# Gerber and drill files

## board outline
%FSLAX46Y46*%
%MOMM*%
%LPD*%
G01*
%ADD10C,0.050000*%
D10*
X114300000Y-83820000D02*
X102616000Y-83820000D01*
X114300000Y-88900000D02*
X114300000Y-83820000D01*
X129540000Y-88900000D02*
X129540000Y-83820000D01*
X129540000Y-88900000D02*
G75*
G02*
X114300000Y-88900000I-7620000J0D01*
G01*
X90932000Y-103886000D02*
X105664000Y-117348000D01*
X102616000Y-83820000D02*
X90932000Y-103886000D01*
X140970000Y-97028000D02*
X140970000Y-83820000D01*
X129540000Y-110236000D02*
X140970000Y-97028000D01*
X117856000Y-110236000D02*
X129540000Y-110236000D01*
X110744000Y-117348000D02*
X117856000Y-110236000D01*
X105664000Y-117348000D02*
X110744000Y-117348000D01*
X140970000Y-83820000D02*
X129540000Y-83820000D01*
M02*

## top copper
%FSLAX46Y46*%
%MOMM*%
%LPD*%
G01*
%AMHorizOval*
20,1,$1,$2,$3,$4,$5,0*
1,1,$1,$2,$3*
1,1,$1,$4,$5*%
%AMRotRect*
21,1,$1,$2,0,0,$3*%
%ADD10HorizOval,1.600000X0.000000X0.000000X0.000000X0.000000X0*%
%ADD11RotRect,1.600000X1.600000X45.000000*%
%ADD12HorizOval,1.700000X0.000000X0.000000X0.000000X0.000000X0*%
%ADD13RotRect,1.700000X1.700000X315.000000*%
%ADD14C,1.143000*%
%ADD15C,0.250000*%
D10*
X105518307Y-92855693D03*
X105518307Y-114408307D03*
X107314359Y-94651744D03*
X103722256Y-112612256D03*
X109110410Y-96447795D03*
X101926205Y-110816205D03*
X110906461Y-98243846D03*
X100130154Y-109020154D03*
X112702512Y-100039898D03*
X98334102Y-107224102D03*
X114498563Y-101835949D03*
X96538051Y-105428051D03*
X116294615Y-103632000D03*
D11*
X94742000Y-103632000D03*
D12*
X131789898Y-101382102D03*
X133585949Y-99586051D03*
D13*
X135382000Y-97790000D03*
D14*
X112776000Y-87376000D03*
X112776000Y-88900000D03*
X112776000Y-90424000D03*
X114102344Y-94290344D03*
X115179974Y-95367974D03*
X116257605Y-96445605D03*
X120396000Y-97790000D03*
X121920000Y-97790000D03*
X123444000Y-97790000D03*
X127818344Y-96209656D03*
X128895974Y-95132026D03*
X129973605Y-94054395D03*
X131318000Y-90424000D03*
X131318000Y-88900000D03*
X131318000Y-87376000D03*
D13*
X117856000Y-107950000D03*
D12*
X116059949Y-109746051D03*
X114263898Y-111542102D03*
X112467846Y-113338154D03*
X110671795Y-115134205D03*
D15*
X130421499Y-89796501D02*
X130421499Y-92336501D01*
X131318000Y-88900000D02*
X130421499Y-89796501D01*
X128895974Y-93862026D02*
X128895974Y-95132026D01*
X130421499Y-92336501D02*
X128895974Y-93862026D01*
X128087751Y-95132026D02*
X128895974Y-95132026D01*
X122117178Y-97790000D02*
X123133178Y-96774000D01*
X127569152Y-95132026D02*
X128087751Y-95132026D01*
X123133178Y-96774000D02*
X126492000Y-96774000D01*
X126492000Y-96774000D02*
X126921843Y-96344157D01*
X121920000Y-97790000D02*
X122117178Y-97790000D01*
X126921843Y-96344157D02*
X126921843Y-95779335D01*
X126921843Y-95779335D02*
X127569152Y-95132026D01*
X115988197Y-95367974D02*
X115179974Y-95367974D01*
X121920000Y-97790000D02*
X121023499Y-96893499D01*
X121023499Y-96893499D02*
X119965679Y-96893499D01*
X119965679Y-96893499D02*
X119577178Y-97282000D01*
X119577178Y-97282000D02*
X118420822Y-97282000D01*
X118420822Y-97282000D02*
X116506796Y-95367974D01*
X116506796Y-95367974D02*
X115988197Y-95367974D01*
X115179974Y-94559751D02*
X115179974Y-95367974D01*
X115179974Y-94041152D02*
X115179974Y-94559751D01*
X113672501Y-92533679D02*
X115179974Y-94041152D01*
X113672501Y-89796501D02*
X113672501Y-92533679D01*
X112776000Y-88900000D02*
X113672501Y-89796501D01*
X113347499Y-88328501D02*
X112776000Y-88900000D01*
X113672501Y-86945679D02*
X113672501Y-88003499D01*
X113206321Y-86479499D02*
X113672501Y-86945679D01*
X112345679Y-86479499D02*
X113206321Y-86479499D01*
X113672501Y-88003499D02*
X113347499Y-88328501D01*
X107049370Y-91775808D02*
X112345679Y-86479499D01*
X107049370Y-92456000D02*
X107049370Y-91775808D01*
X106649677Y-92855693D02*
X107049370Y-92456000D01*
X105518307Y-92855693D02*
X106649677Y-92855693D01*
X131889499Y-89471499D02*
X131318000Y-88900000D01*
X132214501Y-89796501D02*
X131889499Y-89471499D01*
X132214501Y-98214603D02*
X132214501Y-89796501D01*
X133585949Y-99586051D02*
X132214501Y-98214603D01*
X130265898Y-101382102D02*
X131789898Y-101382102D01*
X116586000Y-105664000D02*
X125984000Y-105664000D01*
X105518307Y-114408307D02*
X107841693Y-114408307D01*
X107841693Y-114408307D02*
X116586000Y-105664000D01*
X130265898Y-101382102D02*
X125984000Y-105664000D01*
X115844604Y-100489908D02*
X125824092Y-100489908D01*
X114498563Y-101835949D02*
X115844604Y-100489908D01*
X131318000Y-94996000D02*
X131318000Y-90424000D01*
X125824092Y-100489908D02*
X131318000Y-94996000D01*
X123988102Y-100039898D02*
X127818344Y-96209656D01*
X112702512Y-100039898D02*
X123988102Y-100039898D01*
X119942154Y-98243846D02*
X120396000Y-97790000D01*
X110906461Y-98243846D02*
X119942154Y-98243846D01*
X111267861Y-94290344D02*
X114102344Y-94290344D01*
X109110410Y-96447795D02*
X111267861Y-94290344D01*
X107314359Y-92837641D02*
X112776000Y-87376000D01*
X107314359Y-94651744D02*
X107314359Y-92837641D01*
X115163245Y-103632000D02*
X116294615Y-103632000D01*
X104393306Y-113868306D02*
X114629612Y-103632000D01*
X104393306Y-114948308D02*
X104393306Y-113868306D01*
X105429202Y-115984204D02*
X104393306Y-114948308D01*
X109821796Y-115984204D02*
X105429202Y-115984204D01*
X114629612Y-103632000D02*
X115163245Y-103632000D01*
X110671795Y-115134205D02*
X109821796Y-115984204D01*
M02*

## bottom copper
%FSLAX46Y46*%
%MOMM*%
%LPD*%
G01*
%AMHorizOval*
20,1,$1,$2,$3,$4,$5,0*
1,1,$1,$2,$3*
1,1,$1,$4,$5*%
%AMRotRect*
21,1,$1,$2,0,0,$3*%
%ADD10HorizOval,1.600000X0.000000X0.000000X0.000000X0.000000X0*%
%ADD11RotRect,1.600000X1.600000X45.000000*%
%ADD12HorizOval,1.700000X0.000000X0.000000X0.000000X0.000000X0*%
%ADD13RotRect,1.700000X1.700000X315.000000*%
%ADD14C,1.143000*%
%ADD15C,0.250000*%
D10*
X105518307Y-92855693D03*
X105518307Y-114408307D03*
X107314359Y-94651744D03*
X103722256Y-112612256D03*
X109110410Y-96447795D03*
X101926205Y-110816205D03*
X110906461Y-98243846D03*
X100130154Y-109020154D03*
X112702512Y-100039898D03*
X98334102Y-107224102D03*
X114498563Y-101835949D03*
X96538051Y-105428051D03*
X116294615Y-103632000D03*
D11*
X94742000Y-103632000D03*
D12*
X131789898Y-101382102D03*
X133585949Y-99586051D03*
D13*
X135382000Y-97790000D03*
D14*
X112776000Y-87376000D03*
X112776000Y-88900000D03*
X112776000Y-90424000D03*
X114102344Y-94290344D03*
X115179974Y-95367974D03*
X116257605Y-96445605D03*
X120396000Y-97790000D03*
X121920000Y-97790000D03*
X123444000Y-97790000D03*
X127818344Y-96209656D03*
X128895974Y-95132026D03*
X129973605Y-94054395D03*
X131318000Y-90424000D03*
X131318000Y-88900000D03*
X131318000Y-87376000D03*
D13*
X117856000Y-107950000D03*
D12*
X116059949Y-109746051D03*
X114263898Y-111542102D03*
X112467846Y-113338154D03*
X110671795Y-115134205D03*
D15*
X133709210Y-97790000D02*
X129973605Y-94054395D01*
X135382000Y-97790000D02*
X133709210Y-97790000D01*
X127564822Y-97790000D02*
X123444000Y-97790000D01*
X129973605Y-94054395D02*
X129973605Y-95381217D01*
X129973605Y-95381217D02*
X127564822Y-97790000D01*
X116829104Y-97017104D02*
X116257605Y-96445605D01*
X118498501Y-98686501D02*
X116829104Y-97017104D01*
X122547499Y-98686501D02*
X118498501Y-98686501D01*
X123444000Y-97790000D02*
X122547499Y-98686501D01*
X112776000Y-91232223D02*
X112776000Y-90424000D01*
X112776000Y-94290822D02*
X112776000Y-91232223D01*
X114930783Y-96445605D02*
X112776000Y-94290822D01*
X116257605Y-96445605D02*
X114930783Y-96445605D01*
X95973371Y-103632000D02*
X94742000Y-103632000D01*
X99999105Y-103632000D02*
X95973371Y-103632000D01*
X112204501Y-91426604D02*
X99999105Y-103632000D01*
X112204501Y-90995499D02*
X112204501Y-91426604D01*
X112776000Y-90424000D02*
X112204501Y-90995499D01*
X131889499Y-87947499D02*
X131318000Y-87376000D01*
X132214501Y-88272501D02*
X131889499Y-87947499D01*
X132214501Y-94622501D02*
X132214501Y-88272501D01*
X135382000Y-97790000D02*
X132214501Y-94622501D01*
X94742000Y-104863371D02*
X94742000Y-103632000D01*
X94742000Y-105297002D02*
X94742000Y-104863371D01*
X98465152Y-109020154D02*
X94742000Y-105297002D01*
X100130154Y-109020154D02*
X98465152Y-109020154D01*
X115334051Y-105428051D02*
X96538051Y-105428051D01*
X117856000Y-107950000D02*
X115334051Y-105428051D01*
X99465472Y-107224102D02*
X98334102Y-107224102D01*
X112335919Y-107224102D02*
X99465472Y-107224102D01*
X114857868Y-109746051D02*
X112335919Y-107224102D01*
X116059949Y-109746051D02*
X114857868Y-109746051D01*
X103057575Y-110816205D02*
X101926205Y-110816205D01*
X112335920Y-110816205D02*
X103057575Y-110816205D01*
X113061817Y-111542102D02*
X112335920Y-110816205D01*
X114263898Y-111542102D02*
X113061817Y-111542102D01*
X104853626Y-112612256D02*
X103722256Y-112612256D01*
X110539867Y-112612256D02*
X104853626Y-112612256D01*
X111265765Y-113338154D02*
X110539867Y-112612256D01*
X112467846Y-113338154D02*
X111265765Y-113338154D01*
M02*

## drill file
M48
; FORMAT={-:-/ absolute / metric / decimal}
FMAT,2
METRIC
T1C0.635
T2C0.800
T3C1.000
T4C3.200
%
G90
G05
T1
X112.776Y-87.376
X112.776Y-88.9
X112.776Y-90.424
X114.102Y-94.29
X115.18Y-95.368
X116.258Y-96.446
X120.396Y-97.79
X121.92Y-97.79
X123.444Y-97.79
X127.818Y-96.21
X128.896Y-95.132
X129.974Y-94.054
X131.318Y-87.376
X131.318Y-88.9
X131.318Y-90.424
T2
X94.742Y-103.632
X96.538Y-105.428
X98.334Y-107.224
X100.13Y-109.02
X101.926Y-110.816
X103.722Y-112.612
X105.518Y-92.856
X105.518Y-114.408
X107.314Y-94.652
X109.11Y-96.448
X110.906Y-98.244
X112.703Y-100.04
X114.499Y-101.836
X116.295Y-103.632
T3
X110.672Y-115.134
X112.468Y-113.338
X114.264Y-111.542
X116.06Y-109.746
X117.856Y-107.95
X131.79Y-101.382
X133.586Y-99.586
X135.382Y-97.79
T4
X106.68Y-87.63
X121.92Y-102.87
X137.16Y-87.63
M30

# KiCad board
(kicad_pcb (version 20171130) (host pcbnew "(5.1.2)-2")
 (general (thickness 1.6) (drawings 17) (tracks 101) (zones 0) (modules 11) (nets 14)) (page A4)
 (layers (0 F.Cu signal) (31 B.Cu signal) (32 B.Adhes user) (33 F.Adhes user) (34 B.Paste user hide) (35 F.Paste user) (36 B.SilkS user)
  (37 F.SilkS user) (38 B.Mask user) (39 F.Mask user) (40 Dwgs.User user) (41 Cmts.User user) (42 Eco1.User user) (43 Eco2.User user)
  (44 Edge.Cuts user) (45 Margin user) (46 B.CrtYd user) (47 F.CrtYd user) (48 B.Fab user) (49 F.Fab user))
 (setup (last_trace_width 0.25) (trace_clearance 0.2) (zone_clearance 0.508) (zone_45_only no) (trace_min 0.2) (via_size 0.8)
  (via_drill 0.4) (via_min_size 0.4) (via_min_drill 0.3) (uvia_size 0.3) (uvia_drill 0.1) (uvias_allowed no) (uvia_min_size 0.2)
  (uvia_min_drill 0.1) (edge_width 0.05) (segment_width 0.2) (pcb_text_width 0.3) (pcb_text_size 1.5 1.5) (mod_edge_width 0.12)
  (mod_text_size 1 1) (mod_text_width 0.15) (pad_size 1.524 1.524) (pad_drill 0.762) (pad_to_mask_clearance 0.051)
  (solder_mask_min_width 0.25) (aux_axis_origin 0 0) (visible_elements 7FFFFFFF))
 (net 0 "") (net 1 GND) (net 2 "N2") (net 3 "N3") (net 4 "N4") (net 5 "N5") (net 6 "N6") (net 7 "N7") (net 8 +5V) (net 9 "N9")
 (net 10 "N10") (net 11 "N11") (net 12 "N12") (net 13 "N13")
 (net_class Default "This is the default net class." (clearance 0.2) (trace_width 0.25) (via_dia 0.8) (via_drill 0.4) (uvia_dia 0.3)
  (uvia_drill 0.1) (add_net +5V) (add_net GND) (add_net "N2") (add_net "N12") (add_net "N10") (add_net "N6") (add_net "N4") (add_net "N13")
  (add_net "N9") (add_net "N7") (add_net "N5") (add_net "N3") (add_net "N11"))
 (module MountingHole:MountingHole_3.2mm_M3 (layer F.Cu) (at 121.92 102.87)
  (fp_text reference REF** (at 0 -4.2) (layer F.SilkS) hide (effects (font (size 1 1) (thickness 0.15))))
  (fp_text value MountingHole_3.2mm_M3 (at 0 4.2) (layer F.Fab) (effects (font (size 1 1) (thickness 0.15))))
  (pad 1 np_thru_hole circle (at 0 0) (size 3.2 3.2) (drill 3.2) (layers *.Cu *.Mask)))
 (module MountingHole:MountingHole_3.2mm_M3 (layer F.Cu) (at 137.16 87.63)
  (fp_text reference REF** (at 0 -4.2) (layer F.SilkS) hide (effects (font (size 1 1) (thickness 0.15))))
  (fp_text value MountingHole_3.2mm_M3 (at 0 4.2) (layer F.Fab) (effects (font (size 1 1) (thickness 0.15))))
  (pad 1 np_thru_hole circle (at 0 0) (size 3.2 3.2) (drill 3.2) (layers *.Cu *.Mask)))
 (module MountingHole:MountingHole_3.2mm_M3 (layer F.Cu) (at 106.68 87.63)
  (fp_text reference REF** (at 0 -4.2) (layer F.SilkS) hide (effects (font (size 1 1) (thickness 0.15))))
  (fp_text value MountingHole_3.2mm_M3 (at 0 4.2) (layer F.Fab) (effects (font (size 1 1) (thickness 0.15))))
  (pad 1 np_thru_hole circle (at 0 0) (size 3.2 3.2) (drill 3.2) (layers *.Cu *.Mask)))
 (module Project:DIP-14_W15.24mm (layer F.Cu) (at 94.742 103.632 45)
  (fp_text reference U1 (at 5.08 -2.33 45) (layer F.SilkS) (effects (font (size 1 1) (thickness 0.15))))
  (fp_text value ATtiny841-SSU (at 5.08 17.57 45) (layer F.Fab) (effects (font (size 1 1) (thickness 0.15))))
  (pad 14 thru_hole oval (at 15.24 0 45) (size 1.6 1.6) (drill 0.8) (layers *.Cu *.Mask) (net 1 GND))
  (pad 7 thru_hole oval (at 0 15.24 45) (size 1.6 1.6) (drill 0.8) (layers *.Cu *.Mask) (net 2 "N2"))
  (pad 13 thru_hole oval (at 15.24 2.54 45) (size 1.6 1.6) (drill 0.8) (layers *.Cu *.Mask) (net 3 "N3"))
  (pad 6 thru_hole oval (at 0 12.7 45) (size 1.6 1.6) (drill 0.8) (layers *.Cu *.Mask) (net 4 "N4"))
  (pad 12 thru_hole oval (at 15.24 5.08 45) (size 1.6 1.6) (drill 0.8) (layers *.Cu *.Mask) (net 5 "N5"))
  (pad 5 thru_hole oval (at 0 10.16 45) (size 1.6 1.6) (drill 0.8) (layers *.Cu *.Mask) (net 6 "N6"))
  (pad 11 thru_hole oval (at 15.24 7.62 45) (size 1.6 1.6) (drill 0.8) (layers *.Cu *.Mask) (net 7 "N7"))
  (pad 4 thru_hole oval (at 0 7.62 45) (size 1.6 1.6) (drill 0.8) (layers *.Cu *.Mask) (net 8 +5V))
  (pad 10 thru_hole oval (at 15.24 10.16 45) (size 1.6 1.6) (drill 0.8) (layers *.Cu *.Mask) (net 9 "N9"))
  (pad 3 thru_hole oval (at 0 5.08 45) (size 1.6 1.6) (drill 0.8) (layers *.Cu *.Mask) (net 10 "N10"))
  (pad 9 thru_hole oval (at 15.24 12.7 45) (size 1.6 1.6) (drill 0.8) (layers *.Cu *.Mask) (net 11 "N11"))
  (pad 2 thru_hole oval (at 0 2.54 45) (size 1.6 1.6) (drill 0.8) (layers *.Cu *.Mask) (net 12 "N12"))
  (pad 8 thru_hole oval (at 15.24 15.24 45) (size 1.6 1.6) (drill 0.8) (layers *.Cu *.Mask) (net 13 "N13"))
  (pad 1 thru_hole rect (at 0 0 45) (size 1.6 1.6) (drill 0.8) (layers *.Cu *.Mask) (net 8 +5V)))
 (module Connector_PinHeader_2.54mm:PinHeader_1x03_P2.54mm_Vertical (layer F.Cu) (at 135.382 97.79 315)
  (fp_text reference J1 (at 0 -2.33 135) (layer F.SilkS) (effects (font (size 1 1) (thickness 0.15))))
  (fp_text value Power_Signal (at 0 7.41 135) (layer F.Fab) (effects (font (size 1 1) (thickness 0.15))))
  (pad 3 thru_hole oval (at 0 5.08 315) (size 1.7 1.7) (drill 1) (layers *.Cu *.Mask) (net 2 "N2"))
  (pad 2 thru_hole oval (at 0 2.54 315) (size 1.7 1.7) (drill 1) (layers *.Cu *.Mask) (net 1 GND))
  (pad 1 thru_hole rect (at 0 0 315) (size 1.7 1.7) (drill 1) (layers *.Cu *.Mask) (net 8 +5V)))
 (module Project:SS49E (layer F.Cu) (at 112.776 90.17 90)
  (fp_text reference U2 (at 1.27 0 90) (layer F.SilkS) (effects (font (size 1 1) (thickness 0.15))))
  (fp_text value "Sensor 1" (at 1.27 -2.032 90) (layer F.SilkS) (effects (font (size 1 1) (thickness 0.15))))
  (pad 3 thru_hole circle (at 2.794 0 90) (size 1.143 1.143) (drill 0.635) (layers *.Cu *.Mask) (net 3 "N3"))
  (pad 2 thru_hole circle (at 1.27 0 90) (size 1.143 1.143) (drill 0.635) (layers *.Cu *.Mask) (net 1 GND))
  (pad 1 thru_hole circle (at -0.254 0 90) (size 1.143 1.143) (drill 0.635) (layers *.Cu *.Mask) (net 8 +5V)))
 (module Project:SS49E (layer F.Cu) (at 116.078 96.266 135)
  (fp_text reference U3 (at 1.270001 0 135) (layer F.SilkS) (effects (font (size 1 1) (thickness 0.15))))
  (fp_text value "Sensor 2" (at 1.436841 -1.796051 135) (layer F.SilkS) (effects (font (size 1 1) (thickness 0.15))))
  (pad 3 thru_hole circle (at 2.794 0 135) (size 1.143 1.143) (drill 0.635) (layers *.Cu *.Mask) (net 5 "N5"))
  (pad 2 thru_hole circle (at 1.27 0 135) (size 1.143 1.143) (drill 0.635) (layers *.Cu *.Mask) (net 1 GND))
  (pad 1 thru_hole circle (at -0.254 0 135) (size 1.143 1.143) (drill 0.635) (layers *.Cu *.Mask) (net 8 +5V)))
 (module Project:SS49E (layer F.Cu) (at 123.19 97.79 180)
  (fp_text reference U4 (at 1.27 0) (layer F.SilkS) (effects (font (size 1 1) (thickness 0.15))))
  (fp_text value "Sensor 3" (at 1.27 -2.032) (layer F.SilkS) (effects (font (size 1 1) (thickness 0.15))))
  (pad 3 thru_hole circle (at 2.794 0 180) (size 1.143 1.143) (drill 0.635) (layers *.Cu *.Mask) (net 7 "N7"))
  (pad 2 thru_hole circle (at 1.27 0 180) (size 1.143 1.143) (drill 0.635) (layers *.Cu *.Mask) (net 1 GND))
  (pad 1 thru_hole circle (at -0.254 0 180) (size 1.143 1.143) (drill 0.635) (layers *.Cu *.Mask) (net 8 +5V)))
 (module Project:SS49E (layer F.Cu) (at 129.794 94.234 225)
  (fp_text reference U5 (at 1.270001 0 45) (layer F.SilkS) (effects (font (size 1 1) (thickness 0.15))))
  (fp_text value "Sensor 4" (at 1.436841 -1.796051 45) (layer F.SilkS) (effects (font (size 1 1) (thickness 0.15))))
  (pad 3 thru_hole circle (at 2.794 0 225) (size 1.143 1.143) (drill 0.635) (layers *.Cu *.Mask) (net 9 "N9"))
  (pad 2 thru_hole circle (at 1.27 0 225) (size 1.143 1.143) (drill 0.635) (layers *.Cu *.Mask) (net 1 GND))
  (pad 1 thru_hole circle (at -0.254 0 225) (size 1.143 1.143) (drill 0.635) (layers *.Cu *.Mask) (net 8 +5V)))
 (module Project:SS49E (layer F.Cu) (at 131.318 87.63 270)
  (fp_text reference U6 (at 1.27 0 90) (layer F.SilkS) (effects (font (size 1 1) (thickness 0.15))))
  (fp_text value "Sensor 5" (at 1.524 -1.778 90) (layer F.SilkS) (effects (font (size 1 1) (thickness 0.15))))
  (pad 3 thru_hole circle (at 2.794 0 270) (size 1.143 1.143) (drill 0.635) (layers *.Cu *.Mask) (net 11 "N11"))
  (pad 2 thru_hole circle (at 1.27 0 270) (size 1.143 1.143) (drill 0.635) (layers *.Cu *.Mask) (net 1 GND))
  (pad 1 thru_hole circle (at -0.254 0 270) (size 1.143 1.143) (drill 0.635) (layers *.Cu *.Mask) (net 8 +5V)))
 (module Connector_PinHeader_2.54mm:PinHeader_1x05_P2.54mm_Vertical (layer F.Cu) (at 117.856 107.95 315)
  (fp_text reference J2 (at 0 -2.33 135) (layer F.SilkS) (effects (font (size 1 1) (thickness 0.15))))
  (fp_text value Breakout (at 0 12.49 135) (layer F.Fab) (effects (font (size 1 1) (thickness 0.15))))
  (pad 1 thru_hole rect (at 0 0 315) (size 1.7 1.7) (drill 1) (layers *.Cu *.Mask) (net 12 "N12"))
  (pad 2 thru_hole oval (at 0 2.54 315) (size 1.7 1.7) (drill 1) (layers *.Cu *.Mask) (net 10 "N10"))
  (pad 3 thru_hole oval (at 0 5.08 315) (size 1.7 1.7) (drill 1) (layers *.Cu *.Mask) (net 6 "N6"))
  (pad 4 thru_hole oval (at 0 7.62 315) (size 1.7 1.7) (drill 1) (layers *.Cu *.Mask) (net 4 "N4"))
  (pad 5 thru_hole oval (at 0 10.16 315) (size 1.7 1.7) (drill 1) (layers *.Cu *.Mask) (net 13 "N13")))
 (gr_line (start 114.3 83.82) (end 102.616 83.82) (layer Edge.Cuts) (width 0.05))
 (gr_line (start 114.3 88.9) (end 114.3 83.82) (layer Edge.Cuts) (width 0.05))
 (gr_line (start 129.54 88.9) (end 129.54 83.82) (layer Edge.Cuts) (width 0.05))
 (gr_arc (start 121.92 88.9) (end 114.3 88.9) (angle -180) (layer Edge.Cuts) (width 0.05))
 (gr_line (start 90.932 103.886) (end 105.664 117.348) (layer Edge.Cuts) (width 0.05))
 (gr_line (start 102.616 83.82) (end 90.932 103.886) (layer Edge.Cuts) (width 0.05))
 (gr_line (start 140.97 97.028) (end 140.97 83.82) (layer Edge.Cuts) (width 0.05))
 (gr_line (start 129.54 110.236) (end 140.97 97.028) (layer Edge.Cuts) (width 0.05))
 (gr_line (start 117.856 110.236) (end 129.54 110.236) (layer Edge.Cuts) (width 0.05))
 (gr_line (start 110.744 117.348) (end 117.856 110.236) (layer Edge.Cuts) (width 0.05))
 (gr_line (start 105.664 117.348) (end 110.744 117.348) (layer Edge.Cuts) (width 0.05))
 (gr_line (start 140.97 83.82) (end 129.54 83.82) (layer Edge.Cuts) (width 0.05))
 (segment (start 133.70921 97.79) (end 129.973605 94.054395) (width 0.25) (layer B.Cu) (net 8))
 (segment (start 135.382 97.79) (end 133.70921 97.79) (width 0.25) (layer B.Cu) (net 8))
 (segment (start 127.564822 97.79) (end 123.444 97.79) (width 0.25) (layer B.Cu) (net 8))
 (segment (start 129.973605 94.054395) (end 129.973605 95.381217) (width 0.25) (layer B.Cu) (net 8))
 (segment (start 129.973605 95.381217) (end 127.564822 97.79) (width 0.25) (layer B.Cu) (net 8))
 (segment (start 116.829104 97.017104) (end 116.257605 96.445605) (width 0.25) (layer B.Cu) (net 8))
 (segment (start 118.498501 98.686501) (end 116.829104 97.017104) (width 0.25) (layer B.Cu) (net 8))
 (segment (start 122.547499 98.686501) (end 118.498501 98.686501) (width 0.25) (layer B.Cu) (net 8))
 (segment (start 123.444 97.79) (end 122.547499 98.686501) (width 0.25) (layer B.Cu) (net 8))
 (segment (start 112.776 91.232223) (end 112.776 90.424) (width 0.25) (layer B.Cu) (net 8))
 (segment (start 112.776 94.290822) (end 112.776 91.232223) (width 0.25) (layer B.Cu) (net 8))
 (segment (start 114.930783 96.445605) (end 112.776 94.290822) (width 0.25) (layer B.Cu) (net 8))
 (segment (start 116.257605 96.445605) (end 114.930783 96.445605) (width 0.25) (layer B.Cu) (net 8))
 (segment (start 95.973371 103.632) (end 94.742 103.632) (width 0.25) (layer B.Cu) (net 8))
 (segment (start 99.999105 103.632) (end 95.973371 103.632) (width 0.25) (layer B.Cu) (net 8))
 (segment (start 112.204501 91.426604) (end 99.999105 103.632) (width 0.25) (layer B.Cu) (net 8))
 (segment (start 112.204501 90.995499) (end 112.204501 91.426604) (width 0.25) (layer B.Cu) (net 8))
 (segment (start 112.776 90.424) (end 112.204501 90.995499) (width 0.25) (layer B.Cu) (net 8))
 (segment (start 131.889499 87.947499) (end 131.318 87.376) (width 0.25) (layer B.Cu) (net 8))
 (segment (start 132.214501 88.272501) (end 131.889499 87.947499) (width 0.25) (layer B.Cu) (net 8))
 (segment (start 132.214501 94.622501) (end 132.214501 88.272501) (width 0.25) (layer B.Cu) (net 8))
 (segment (start 135.382 97.79) (end 132.214501 94.622501) (width 0.25) (layer B.Cu) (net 8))
 (segment (start 94.742 104.863371) (end 94.742 103.632) (width 0.25) (layer B.Cu) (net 8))
 (segment (start 94.742 105.297002) (end 94.742 104.863371) (width 0.25) (layer B.Cu) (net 8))
 (segment (start 98.465152 109.020154) (end 94.742 105.297002) (width 0.25) (layer B.Cu) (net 8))
 (segment (start 100.130154 109.020154) (end 98.465152 109.020154) (width 0.25) (layer B.Cu) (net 8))
 (segment (start 130.421499 89.796501) (end 130.421499 92.336501) (width 0.25) (layer F.Cu) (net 1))
 (segment (start 131.318 88.9) (end 130.421499 89.796501) (width 0.25) (layer F.Cu) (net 1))
 (segment (start 128.895974 93.862026) (end 128.895974 95.132026) (width 0.25) (layer F.Cu) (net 1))
 (segment (start 130.421499 92.336501) (end 128.895974 93.862026) (width 0.25) (layer F.Cu) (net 1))
 (segment (start 128.087751 95.132026) (end 128.895974 95.132026) (width 0.25) (layer F.Cu) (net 1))
 (segment (start 122.117178 97.79) (end 123.133178 96.774) (width 0.25) (layer F.Cu) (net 1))
 (segment (start 127.569152 95.132026) (end 128.087751 95.132026) (width 0.25) (layer F.Cu) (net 1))
 (segment (start 123.133178 96.774) (end 126.492 96.774) (width 0.25) (layer F.Cu) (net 1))
 (segment (start 126.492 96.774) (end 126.921843 96.344157) (width 0.25) (layer F.Cu) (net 1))
 (segment (start 121.92 97.79) (end 122.117178 97.79) (width 0.25) (layer F.Cu) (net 1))
 (segment (start 126.921843 96.344157) (end 126.921843 95.779335) (width 0.25) (layer F.Cu) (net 1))
 (segment (start 126.921843 95.779335) (end 127.569152 95.132026) (width 0.25) (layer F.Cu) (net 1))
 (segment (start 115.988197 95.367974) (end 115.179974 95.367974) (width 0.25) (layer F.Cu) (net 1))
 (segment (start 121.92 97.79) (end 121.023499 96.893499) (width 0.25) (layer F.Cu) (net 1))
 (segment (start 121.023499 96.893499) (end 119.965679 96.893499) (width 0.25) (layer F.Cu) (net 1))
 (segment (start 119.965679 96.893499) (end 119.577178 97.282) (width 0.25) (layer F.Cu) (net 1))
 (segment (start 119.577178 97.282) (end 118.420822 97.282) (width 0.25) (layer F.Cu) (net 1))
 (segment (start 118.420822 97.282) (end 116.506796 95.367974) (width 0.25) (layer F.Cu) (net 1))
 (segment (start 116.506796 95.367974) (end 115.988197 95.367974) (width 0.25) (layer F.Cu) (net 1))
 (segment (start 115.179974 94.559751) (end 115.179974 95.367974) (width 0.25) (layer F.Cu) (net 1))
 (segment (start 115.179974 94.041152) (end 115.179974 94.559751) (width 0.25) (layer F.Cu) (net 1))
 (segment (start 113.672501 92.533679) (end 115.179974 94.041152) (width 0.25) (layer F.Cu) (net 1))
 (segment (start 113.672501 89.796501) (end 113.672501 92.533679) (width 0.25) (layer F.Cu) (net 1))
 (segment (start 112.776 88.9) (end 113.672501 89.796501) (width 0.25) (layer F.Cu) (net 1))
 (segment (start 113.347499 88.328501) (end 112.776 88.9) (width 0.25) (layer F.Cu) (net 1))
 (segment (start 113.672501 86.945679) (end 113.672501 88.003499) (width 0.25) (layer F.Cu) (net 1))
 (segment (start 113.206321 86.479499) (end 113.672501 86.945679) (width 0.25) (layer F.Cu) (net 1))
 (segment (start 112.345679 86.479499) (end 113.206321 86.479499) (width 0.25) (layer F.Cu) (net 1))
 (segment (start 113.672501 88.003499) (end 113.347499 88.328501) (width 0.25) (layer F.Cu) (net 1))
 (segment (start 107.04937 91.775808) (end 112.345679 86.479499) (width 0.25) (layer F.Cu) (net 1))
 (segment (start 107.04937 92.456) (end 107.04937 91.775808) (width 0.25) (layer F.Cu) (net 1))
 (segment (start 106.649677 92.855693) (end 107.04937 92.456) (width 0.25) (layer F.Cu) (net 1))
 (segment (start 105.518307 92.855693) (end 106.649677 92.855693) (width 0.25) (layer F.Cu) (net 1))
 (segment (start 131.889499 89.471499) (end 131.318 88.9) (width 0.25) (layer F.Cu) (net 1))
 (segment (start 132.214501 89.796501) (end 131.889499 89.471499) (width 0.25) (layer F.Cu) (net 1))
 (segment (start 132.214501 98.214603) (end 132.214501 89.796501) (width 0.25) (layer F.Cu) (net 1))
 (segment (start 133.585949 99.586051) (end 132.214501 98.214603) (width 0.25) (layer F.Cu) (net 1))
 (segment (start 130.265898 101.382102) (end 131.789898 101.382102) (width 0.25) (layer F.Cu) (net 2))
 (segment (start 116.586 105.664) (end 125.984 105.664) (width 0.25) (layer F.Cu) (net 2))
 (segment (start 105.518307 114.408307) (end 107.841693 114.408307) (width 0.25) (layer F.Cu) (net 2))
 (segment (start 107.841693 114.408307) (end 116.586 105.664) (width 0.25) (layer F.Cu) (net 2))
 (segment (start 130.265898 101.382102) (end 125.984 105.664) (width 0.25) (layer F.Cu) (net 2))
 (segment (start 115.844604 100.489908) (end 125.824092 100.489908) (width 0.25) (layer F.Cu) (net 11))
 (segment (start 114.498563 101.835949) (end 115.844604 100.489908) (width 0.25) (layer F.Cu) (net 11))
 (segment (start 131.318 94.996) (end 131.318 90.424) (width 0.25) (layer F.Cu) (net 11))
 (segment (start 125.824092 100.489908) (end 131.318 94.996) (width 0.25) (layer F.Cu) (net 11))
 (segment (start 123.988102 100.039898) (end 127.818344 96.209656) (width 0.25) (layer F.Cu) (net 9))
 (segment (start 112.702512 100.039898) (end 123.988102 100.039898) (width 0.25) (layer F.Cu) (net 9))
 (segment (start 119.942154 98.243846) (end 120.396 97.79) (width 0.25) (layer F.Cu) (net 7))
 (segment (start 110.906461 98.243846) (end 119.942154 98.243846) (width 0.25) (layer F.Cu) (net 7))
 (segment (start 111.267861 94.290344) (end 114.102344 94.290344) (width 0.25) (layer F.Cu) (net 5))
 (segment (start 109.11041 96.447795) (end 111.267861 94.290344) (width 0.25) (layer F.Cu) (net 5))
 (segment (start 107.314359 92.837641) (end 112.776 87.376) (width 0.25) (layer F.Cu) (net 3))
 (segment (start 107.314359 94.651744) (end 107.314359 92.837641) (width 0.25) (layer F.Cu) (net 3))
 (segment (start 115.334051 105.428051) (end 96.538051 105.428051) (width 0.25) (layer B.Cu) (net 12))
 (segment (start 117.856 107.95) (end 115.334051 105.428051) (width 0.25) (layer B.Cu) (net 12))
 (segment (start 99.465472 107.224102) (end 98.334102 107.224102) (width 0.25) (layer B.Cu) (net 10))
 (segment (start 112.335919 107.224102) (end 99.465472 107.224102) (width 0.25) (layer B.Cu) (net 10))
 (segment (start 114.857868 109.746051) (end 112.335919 107.224102) (width 0.25) (layer B.Cu) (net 10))
 (segment (start 116.059949 109.746051) (end 114.857868 109.746051) (width 0.25) (layer B.Cu) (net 10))
 (segment (start 103.057575 110.816205) (end 101.926205 110.816205) (width 0.25) (layer B.Cu) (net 6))
 (segment (start 112.33592 110.816205) (end 103.057575 110.816205) (width 0.25) (layer B.Cu) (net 6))
 (segment (start 113.061817 111.542102) (end 112.33592 110.816205) (width 0.25) (layer B.Cu) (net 6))
 (segment (start 114.263898 111.542102) (end 113.061817 111.542102) (width 0.25) (layer B.Cu) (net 6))
 (segment (start 104.853626 112.612256) (end 103.722256 112.612256) (width 0.25) (layer B.Cu) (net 4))
 (segment (start 110.539867 112.612256) (end 104.853626 112.612256) (width 0.25) (layer B.Cu) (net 4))
 (segment (start 111.265765 113.338154) (end 110.539867 112.612256) (width 0.25) (layer B.Cu) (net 4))
 (segment (start 112.467846 113.338154) (end 111.265765 113.338154) (width 0.25) (layer B.Cu) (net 4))
 (segment (start 115.163245 103.632) (end 116.294615 103.632) (width 0.25) (layer F.Cu) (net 13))
 (segment (start 104.393306 113.868306) (end 114.629612 103.632) (width 0.25) (layer F.Cu) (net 13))
 (segment (start 104.393306 114.948308) (end 104.393306 113.868306) (width 0.25) (layer F.Cu) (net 13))
 (segment (start 105.429202 115.984204) (end 104.393306 114.948308) (width 0.25) (layer F.Cu) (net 13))
 (segment (start 109.821796 115.984204) (end 105.429202 115.984204) (width 0.25) (layer F.Cu) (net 13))
 (segment (start 114.629612 103.632) (end 115.163245 103.632) (width 0.25) (layer F.Cu) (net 13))
 (segment (start 110.671795 115.134205) (end 109.821796 115.984204) (width 0.25) (layer F.Cu) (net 13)))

